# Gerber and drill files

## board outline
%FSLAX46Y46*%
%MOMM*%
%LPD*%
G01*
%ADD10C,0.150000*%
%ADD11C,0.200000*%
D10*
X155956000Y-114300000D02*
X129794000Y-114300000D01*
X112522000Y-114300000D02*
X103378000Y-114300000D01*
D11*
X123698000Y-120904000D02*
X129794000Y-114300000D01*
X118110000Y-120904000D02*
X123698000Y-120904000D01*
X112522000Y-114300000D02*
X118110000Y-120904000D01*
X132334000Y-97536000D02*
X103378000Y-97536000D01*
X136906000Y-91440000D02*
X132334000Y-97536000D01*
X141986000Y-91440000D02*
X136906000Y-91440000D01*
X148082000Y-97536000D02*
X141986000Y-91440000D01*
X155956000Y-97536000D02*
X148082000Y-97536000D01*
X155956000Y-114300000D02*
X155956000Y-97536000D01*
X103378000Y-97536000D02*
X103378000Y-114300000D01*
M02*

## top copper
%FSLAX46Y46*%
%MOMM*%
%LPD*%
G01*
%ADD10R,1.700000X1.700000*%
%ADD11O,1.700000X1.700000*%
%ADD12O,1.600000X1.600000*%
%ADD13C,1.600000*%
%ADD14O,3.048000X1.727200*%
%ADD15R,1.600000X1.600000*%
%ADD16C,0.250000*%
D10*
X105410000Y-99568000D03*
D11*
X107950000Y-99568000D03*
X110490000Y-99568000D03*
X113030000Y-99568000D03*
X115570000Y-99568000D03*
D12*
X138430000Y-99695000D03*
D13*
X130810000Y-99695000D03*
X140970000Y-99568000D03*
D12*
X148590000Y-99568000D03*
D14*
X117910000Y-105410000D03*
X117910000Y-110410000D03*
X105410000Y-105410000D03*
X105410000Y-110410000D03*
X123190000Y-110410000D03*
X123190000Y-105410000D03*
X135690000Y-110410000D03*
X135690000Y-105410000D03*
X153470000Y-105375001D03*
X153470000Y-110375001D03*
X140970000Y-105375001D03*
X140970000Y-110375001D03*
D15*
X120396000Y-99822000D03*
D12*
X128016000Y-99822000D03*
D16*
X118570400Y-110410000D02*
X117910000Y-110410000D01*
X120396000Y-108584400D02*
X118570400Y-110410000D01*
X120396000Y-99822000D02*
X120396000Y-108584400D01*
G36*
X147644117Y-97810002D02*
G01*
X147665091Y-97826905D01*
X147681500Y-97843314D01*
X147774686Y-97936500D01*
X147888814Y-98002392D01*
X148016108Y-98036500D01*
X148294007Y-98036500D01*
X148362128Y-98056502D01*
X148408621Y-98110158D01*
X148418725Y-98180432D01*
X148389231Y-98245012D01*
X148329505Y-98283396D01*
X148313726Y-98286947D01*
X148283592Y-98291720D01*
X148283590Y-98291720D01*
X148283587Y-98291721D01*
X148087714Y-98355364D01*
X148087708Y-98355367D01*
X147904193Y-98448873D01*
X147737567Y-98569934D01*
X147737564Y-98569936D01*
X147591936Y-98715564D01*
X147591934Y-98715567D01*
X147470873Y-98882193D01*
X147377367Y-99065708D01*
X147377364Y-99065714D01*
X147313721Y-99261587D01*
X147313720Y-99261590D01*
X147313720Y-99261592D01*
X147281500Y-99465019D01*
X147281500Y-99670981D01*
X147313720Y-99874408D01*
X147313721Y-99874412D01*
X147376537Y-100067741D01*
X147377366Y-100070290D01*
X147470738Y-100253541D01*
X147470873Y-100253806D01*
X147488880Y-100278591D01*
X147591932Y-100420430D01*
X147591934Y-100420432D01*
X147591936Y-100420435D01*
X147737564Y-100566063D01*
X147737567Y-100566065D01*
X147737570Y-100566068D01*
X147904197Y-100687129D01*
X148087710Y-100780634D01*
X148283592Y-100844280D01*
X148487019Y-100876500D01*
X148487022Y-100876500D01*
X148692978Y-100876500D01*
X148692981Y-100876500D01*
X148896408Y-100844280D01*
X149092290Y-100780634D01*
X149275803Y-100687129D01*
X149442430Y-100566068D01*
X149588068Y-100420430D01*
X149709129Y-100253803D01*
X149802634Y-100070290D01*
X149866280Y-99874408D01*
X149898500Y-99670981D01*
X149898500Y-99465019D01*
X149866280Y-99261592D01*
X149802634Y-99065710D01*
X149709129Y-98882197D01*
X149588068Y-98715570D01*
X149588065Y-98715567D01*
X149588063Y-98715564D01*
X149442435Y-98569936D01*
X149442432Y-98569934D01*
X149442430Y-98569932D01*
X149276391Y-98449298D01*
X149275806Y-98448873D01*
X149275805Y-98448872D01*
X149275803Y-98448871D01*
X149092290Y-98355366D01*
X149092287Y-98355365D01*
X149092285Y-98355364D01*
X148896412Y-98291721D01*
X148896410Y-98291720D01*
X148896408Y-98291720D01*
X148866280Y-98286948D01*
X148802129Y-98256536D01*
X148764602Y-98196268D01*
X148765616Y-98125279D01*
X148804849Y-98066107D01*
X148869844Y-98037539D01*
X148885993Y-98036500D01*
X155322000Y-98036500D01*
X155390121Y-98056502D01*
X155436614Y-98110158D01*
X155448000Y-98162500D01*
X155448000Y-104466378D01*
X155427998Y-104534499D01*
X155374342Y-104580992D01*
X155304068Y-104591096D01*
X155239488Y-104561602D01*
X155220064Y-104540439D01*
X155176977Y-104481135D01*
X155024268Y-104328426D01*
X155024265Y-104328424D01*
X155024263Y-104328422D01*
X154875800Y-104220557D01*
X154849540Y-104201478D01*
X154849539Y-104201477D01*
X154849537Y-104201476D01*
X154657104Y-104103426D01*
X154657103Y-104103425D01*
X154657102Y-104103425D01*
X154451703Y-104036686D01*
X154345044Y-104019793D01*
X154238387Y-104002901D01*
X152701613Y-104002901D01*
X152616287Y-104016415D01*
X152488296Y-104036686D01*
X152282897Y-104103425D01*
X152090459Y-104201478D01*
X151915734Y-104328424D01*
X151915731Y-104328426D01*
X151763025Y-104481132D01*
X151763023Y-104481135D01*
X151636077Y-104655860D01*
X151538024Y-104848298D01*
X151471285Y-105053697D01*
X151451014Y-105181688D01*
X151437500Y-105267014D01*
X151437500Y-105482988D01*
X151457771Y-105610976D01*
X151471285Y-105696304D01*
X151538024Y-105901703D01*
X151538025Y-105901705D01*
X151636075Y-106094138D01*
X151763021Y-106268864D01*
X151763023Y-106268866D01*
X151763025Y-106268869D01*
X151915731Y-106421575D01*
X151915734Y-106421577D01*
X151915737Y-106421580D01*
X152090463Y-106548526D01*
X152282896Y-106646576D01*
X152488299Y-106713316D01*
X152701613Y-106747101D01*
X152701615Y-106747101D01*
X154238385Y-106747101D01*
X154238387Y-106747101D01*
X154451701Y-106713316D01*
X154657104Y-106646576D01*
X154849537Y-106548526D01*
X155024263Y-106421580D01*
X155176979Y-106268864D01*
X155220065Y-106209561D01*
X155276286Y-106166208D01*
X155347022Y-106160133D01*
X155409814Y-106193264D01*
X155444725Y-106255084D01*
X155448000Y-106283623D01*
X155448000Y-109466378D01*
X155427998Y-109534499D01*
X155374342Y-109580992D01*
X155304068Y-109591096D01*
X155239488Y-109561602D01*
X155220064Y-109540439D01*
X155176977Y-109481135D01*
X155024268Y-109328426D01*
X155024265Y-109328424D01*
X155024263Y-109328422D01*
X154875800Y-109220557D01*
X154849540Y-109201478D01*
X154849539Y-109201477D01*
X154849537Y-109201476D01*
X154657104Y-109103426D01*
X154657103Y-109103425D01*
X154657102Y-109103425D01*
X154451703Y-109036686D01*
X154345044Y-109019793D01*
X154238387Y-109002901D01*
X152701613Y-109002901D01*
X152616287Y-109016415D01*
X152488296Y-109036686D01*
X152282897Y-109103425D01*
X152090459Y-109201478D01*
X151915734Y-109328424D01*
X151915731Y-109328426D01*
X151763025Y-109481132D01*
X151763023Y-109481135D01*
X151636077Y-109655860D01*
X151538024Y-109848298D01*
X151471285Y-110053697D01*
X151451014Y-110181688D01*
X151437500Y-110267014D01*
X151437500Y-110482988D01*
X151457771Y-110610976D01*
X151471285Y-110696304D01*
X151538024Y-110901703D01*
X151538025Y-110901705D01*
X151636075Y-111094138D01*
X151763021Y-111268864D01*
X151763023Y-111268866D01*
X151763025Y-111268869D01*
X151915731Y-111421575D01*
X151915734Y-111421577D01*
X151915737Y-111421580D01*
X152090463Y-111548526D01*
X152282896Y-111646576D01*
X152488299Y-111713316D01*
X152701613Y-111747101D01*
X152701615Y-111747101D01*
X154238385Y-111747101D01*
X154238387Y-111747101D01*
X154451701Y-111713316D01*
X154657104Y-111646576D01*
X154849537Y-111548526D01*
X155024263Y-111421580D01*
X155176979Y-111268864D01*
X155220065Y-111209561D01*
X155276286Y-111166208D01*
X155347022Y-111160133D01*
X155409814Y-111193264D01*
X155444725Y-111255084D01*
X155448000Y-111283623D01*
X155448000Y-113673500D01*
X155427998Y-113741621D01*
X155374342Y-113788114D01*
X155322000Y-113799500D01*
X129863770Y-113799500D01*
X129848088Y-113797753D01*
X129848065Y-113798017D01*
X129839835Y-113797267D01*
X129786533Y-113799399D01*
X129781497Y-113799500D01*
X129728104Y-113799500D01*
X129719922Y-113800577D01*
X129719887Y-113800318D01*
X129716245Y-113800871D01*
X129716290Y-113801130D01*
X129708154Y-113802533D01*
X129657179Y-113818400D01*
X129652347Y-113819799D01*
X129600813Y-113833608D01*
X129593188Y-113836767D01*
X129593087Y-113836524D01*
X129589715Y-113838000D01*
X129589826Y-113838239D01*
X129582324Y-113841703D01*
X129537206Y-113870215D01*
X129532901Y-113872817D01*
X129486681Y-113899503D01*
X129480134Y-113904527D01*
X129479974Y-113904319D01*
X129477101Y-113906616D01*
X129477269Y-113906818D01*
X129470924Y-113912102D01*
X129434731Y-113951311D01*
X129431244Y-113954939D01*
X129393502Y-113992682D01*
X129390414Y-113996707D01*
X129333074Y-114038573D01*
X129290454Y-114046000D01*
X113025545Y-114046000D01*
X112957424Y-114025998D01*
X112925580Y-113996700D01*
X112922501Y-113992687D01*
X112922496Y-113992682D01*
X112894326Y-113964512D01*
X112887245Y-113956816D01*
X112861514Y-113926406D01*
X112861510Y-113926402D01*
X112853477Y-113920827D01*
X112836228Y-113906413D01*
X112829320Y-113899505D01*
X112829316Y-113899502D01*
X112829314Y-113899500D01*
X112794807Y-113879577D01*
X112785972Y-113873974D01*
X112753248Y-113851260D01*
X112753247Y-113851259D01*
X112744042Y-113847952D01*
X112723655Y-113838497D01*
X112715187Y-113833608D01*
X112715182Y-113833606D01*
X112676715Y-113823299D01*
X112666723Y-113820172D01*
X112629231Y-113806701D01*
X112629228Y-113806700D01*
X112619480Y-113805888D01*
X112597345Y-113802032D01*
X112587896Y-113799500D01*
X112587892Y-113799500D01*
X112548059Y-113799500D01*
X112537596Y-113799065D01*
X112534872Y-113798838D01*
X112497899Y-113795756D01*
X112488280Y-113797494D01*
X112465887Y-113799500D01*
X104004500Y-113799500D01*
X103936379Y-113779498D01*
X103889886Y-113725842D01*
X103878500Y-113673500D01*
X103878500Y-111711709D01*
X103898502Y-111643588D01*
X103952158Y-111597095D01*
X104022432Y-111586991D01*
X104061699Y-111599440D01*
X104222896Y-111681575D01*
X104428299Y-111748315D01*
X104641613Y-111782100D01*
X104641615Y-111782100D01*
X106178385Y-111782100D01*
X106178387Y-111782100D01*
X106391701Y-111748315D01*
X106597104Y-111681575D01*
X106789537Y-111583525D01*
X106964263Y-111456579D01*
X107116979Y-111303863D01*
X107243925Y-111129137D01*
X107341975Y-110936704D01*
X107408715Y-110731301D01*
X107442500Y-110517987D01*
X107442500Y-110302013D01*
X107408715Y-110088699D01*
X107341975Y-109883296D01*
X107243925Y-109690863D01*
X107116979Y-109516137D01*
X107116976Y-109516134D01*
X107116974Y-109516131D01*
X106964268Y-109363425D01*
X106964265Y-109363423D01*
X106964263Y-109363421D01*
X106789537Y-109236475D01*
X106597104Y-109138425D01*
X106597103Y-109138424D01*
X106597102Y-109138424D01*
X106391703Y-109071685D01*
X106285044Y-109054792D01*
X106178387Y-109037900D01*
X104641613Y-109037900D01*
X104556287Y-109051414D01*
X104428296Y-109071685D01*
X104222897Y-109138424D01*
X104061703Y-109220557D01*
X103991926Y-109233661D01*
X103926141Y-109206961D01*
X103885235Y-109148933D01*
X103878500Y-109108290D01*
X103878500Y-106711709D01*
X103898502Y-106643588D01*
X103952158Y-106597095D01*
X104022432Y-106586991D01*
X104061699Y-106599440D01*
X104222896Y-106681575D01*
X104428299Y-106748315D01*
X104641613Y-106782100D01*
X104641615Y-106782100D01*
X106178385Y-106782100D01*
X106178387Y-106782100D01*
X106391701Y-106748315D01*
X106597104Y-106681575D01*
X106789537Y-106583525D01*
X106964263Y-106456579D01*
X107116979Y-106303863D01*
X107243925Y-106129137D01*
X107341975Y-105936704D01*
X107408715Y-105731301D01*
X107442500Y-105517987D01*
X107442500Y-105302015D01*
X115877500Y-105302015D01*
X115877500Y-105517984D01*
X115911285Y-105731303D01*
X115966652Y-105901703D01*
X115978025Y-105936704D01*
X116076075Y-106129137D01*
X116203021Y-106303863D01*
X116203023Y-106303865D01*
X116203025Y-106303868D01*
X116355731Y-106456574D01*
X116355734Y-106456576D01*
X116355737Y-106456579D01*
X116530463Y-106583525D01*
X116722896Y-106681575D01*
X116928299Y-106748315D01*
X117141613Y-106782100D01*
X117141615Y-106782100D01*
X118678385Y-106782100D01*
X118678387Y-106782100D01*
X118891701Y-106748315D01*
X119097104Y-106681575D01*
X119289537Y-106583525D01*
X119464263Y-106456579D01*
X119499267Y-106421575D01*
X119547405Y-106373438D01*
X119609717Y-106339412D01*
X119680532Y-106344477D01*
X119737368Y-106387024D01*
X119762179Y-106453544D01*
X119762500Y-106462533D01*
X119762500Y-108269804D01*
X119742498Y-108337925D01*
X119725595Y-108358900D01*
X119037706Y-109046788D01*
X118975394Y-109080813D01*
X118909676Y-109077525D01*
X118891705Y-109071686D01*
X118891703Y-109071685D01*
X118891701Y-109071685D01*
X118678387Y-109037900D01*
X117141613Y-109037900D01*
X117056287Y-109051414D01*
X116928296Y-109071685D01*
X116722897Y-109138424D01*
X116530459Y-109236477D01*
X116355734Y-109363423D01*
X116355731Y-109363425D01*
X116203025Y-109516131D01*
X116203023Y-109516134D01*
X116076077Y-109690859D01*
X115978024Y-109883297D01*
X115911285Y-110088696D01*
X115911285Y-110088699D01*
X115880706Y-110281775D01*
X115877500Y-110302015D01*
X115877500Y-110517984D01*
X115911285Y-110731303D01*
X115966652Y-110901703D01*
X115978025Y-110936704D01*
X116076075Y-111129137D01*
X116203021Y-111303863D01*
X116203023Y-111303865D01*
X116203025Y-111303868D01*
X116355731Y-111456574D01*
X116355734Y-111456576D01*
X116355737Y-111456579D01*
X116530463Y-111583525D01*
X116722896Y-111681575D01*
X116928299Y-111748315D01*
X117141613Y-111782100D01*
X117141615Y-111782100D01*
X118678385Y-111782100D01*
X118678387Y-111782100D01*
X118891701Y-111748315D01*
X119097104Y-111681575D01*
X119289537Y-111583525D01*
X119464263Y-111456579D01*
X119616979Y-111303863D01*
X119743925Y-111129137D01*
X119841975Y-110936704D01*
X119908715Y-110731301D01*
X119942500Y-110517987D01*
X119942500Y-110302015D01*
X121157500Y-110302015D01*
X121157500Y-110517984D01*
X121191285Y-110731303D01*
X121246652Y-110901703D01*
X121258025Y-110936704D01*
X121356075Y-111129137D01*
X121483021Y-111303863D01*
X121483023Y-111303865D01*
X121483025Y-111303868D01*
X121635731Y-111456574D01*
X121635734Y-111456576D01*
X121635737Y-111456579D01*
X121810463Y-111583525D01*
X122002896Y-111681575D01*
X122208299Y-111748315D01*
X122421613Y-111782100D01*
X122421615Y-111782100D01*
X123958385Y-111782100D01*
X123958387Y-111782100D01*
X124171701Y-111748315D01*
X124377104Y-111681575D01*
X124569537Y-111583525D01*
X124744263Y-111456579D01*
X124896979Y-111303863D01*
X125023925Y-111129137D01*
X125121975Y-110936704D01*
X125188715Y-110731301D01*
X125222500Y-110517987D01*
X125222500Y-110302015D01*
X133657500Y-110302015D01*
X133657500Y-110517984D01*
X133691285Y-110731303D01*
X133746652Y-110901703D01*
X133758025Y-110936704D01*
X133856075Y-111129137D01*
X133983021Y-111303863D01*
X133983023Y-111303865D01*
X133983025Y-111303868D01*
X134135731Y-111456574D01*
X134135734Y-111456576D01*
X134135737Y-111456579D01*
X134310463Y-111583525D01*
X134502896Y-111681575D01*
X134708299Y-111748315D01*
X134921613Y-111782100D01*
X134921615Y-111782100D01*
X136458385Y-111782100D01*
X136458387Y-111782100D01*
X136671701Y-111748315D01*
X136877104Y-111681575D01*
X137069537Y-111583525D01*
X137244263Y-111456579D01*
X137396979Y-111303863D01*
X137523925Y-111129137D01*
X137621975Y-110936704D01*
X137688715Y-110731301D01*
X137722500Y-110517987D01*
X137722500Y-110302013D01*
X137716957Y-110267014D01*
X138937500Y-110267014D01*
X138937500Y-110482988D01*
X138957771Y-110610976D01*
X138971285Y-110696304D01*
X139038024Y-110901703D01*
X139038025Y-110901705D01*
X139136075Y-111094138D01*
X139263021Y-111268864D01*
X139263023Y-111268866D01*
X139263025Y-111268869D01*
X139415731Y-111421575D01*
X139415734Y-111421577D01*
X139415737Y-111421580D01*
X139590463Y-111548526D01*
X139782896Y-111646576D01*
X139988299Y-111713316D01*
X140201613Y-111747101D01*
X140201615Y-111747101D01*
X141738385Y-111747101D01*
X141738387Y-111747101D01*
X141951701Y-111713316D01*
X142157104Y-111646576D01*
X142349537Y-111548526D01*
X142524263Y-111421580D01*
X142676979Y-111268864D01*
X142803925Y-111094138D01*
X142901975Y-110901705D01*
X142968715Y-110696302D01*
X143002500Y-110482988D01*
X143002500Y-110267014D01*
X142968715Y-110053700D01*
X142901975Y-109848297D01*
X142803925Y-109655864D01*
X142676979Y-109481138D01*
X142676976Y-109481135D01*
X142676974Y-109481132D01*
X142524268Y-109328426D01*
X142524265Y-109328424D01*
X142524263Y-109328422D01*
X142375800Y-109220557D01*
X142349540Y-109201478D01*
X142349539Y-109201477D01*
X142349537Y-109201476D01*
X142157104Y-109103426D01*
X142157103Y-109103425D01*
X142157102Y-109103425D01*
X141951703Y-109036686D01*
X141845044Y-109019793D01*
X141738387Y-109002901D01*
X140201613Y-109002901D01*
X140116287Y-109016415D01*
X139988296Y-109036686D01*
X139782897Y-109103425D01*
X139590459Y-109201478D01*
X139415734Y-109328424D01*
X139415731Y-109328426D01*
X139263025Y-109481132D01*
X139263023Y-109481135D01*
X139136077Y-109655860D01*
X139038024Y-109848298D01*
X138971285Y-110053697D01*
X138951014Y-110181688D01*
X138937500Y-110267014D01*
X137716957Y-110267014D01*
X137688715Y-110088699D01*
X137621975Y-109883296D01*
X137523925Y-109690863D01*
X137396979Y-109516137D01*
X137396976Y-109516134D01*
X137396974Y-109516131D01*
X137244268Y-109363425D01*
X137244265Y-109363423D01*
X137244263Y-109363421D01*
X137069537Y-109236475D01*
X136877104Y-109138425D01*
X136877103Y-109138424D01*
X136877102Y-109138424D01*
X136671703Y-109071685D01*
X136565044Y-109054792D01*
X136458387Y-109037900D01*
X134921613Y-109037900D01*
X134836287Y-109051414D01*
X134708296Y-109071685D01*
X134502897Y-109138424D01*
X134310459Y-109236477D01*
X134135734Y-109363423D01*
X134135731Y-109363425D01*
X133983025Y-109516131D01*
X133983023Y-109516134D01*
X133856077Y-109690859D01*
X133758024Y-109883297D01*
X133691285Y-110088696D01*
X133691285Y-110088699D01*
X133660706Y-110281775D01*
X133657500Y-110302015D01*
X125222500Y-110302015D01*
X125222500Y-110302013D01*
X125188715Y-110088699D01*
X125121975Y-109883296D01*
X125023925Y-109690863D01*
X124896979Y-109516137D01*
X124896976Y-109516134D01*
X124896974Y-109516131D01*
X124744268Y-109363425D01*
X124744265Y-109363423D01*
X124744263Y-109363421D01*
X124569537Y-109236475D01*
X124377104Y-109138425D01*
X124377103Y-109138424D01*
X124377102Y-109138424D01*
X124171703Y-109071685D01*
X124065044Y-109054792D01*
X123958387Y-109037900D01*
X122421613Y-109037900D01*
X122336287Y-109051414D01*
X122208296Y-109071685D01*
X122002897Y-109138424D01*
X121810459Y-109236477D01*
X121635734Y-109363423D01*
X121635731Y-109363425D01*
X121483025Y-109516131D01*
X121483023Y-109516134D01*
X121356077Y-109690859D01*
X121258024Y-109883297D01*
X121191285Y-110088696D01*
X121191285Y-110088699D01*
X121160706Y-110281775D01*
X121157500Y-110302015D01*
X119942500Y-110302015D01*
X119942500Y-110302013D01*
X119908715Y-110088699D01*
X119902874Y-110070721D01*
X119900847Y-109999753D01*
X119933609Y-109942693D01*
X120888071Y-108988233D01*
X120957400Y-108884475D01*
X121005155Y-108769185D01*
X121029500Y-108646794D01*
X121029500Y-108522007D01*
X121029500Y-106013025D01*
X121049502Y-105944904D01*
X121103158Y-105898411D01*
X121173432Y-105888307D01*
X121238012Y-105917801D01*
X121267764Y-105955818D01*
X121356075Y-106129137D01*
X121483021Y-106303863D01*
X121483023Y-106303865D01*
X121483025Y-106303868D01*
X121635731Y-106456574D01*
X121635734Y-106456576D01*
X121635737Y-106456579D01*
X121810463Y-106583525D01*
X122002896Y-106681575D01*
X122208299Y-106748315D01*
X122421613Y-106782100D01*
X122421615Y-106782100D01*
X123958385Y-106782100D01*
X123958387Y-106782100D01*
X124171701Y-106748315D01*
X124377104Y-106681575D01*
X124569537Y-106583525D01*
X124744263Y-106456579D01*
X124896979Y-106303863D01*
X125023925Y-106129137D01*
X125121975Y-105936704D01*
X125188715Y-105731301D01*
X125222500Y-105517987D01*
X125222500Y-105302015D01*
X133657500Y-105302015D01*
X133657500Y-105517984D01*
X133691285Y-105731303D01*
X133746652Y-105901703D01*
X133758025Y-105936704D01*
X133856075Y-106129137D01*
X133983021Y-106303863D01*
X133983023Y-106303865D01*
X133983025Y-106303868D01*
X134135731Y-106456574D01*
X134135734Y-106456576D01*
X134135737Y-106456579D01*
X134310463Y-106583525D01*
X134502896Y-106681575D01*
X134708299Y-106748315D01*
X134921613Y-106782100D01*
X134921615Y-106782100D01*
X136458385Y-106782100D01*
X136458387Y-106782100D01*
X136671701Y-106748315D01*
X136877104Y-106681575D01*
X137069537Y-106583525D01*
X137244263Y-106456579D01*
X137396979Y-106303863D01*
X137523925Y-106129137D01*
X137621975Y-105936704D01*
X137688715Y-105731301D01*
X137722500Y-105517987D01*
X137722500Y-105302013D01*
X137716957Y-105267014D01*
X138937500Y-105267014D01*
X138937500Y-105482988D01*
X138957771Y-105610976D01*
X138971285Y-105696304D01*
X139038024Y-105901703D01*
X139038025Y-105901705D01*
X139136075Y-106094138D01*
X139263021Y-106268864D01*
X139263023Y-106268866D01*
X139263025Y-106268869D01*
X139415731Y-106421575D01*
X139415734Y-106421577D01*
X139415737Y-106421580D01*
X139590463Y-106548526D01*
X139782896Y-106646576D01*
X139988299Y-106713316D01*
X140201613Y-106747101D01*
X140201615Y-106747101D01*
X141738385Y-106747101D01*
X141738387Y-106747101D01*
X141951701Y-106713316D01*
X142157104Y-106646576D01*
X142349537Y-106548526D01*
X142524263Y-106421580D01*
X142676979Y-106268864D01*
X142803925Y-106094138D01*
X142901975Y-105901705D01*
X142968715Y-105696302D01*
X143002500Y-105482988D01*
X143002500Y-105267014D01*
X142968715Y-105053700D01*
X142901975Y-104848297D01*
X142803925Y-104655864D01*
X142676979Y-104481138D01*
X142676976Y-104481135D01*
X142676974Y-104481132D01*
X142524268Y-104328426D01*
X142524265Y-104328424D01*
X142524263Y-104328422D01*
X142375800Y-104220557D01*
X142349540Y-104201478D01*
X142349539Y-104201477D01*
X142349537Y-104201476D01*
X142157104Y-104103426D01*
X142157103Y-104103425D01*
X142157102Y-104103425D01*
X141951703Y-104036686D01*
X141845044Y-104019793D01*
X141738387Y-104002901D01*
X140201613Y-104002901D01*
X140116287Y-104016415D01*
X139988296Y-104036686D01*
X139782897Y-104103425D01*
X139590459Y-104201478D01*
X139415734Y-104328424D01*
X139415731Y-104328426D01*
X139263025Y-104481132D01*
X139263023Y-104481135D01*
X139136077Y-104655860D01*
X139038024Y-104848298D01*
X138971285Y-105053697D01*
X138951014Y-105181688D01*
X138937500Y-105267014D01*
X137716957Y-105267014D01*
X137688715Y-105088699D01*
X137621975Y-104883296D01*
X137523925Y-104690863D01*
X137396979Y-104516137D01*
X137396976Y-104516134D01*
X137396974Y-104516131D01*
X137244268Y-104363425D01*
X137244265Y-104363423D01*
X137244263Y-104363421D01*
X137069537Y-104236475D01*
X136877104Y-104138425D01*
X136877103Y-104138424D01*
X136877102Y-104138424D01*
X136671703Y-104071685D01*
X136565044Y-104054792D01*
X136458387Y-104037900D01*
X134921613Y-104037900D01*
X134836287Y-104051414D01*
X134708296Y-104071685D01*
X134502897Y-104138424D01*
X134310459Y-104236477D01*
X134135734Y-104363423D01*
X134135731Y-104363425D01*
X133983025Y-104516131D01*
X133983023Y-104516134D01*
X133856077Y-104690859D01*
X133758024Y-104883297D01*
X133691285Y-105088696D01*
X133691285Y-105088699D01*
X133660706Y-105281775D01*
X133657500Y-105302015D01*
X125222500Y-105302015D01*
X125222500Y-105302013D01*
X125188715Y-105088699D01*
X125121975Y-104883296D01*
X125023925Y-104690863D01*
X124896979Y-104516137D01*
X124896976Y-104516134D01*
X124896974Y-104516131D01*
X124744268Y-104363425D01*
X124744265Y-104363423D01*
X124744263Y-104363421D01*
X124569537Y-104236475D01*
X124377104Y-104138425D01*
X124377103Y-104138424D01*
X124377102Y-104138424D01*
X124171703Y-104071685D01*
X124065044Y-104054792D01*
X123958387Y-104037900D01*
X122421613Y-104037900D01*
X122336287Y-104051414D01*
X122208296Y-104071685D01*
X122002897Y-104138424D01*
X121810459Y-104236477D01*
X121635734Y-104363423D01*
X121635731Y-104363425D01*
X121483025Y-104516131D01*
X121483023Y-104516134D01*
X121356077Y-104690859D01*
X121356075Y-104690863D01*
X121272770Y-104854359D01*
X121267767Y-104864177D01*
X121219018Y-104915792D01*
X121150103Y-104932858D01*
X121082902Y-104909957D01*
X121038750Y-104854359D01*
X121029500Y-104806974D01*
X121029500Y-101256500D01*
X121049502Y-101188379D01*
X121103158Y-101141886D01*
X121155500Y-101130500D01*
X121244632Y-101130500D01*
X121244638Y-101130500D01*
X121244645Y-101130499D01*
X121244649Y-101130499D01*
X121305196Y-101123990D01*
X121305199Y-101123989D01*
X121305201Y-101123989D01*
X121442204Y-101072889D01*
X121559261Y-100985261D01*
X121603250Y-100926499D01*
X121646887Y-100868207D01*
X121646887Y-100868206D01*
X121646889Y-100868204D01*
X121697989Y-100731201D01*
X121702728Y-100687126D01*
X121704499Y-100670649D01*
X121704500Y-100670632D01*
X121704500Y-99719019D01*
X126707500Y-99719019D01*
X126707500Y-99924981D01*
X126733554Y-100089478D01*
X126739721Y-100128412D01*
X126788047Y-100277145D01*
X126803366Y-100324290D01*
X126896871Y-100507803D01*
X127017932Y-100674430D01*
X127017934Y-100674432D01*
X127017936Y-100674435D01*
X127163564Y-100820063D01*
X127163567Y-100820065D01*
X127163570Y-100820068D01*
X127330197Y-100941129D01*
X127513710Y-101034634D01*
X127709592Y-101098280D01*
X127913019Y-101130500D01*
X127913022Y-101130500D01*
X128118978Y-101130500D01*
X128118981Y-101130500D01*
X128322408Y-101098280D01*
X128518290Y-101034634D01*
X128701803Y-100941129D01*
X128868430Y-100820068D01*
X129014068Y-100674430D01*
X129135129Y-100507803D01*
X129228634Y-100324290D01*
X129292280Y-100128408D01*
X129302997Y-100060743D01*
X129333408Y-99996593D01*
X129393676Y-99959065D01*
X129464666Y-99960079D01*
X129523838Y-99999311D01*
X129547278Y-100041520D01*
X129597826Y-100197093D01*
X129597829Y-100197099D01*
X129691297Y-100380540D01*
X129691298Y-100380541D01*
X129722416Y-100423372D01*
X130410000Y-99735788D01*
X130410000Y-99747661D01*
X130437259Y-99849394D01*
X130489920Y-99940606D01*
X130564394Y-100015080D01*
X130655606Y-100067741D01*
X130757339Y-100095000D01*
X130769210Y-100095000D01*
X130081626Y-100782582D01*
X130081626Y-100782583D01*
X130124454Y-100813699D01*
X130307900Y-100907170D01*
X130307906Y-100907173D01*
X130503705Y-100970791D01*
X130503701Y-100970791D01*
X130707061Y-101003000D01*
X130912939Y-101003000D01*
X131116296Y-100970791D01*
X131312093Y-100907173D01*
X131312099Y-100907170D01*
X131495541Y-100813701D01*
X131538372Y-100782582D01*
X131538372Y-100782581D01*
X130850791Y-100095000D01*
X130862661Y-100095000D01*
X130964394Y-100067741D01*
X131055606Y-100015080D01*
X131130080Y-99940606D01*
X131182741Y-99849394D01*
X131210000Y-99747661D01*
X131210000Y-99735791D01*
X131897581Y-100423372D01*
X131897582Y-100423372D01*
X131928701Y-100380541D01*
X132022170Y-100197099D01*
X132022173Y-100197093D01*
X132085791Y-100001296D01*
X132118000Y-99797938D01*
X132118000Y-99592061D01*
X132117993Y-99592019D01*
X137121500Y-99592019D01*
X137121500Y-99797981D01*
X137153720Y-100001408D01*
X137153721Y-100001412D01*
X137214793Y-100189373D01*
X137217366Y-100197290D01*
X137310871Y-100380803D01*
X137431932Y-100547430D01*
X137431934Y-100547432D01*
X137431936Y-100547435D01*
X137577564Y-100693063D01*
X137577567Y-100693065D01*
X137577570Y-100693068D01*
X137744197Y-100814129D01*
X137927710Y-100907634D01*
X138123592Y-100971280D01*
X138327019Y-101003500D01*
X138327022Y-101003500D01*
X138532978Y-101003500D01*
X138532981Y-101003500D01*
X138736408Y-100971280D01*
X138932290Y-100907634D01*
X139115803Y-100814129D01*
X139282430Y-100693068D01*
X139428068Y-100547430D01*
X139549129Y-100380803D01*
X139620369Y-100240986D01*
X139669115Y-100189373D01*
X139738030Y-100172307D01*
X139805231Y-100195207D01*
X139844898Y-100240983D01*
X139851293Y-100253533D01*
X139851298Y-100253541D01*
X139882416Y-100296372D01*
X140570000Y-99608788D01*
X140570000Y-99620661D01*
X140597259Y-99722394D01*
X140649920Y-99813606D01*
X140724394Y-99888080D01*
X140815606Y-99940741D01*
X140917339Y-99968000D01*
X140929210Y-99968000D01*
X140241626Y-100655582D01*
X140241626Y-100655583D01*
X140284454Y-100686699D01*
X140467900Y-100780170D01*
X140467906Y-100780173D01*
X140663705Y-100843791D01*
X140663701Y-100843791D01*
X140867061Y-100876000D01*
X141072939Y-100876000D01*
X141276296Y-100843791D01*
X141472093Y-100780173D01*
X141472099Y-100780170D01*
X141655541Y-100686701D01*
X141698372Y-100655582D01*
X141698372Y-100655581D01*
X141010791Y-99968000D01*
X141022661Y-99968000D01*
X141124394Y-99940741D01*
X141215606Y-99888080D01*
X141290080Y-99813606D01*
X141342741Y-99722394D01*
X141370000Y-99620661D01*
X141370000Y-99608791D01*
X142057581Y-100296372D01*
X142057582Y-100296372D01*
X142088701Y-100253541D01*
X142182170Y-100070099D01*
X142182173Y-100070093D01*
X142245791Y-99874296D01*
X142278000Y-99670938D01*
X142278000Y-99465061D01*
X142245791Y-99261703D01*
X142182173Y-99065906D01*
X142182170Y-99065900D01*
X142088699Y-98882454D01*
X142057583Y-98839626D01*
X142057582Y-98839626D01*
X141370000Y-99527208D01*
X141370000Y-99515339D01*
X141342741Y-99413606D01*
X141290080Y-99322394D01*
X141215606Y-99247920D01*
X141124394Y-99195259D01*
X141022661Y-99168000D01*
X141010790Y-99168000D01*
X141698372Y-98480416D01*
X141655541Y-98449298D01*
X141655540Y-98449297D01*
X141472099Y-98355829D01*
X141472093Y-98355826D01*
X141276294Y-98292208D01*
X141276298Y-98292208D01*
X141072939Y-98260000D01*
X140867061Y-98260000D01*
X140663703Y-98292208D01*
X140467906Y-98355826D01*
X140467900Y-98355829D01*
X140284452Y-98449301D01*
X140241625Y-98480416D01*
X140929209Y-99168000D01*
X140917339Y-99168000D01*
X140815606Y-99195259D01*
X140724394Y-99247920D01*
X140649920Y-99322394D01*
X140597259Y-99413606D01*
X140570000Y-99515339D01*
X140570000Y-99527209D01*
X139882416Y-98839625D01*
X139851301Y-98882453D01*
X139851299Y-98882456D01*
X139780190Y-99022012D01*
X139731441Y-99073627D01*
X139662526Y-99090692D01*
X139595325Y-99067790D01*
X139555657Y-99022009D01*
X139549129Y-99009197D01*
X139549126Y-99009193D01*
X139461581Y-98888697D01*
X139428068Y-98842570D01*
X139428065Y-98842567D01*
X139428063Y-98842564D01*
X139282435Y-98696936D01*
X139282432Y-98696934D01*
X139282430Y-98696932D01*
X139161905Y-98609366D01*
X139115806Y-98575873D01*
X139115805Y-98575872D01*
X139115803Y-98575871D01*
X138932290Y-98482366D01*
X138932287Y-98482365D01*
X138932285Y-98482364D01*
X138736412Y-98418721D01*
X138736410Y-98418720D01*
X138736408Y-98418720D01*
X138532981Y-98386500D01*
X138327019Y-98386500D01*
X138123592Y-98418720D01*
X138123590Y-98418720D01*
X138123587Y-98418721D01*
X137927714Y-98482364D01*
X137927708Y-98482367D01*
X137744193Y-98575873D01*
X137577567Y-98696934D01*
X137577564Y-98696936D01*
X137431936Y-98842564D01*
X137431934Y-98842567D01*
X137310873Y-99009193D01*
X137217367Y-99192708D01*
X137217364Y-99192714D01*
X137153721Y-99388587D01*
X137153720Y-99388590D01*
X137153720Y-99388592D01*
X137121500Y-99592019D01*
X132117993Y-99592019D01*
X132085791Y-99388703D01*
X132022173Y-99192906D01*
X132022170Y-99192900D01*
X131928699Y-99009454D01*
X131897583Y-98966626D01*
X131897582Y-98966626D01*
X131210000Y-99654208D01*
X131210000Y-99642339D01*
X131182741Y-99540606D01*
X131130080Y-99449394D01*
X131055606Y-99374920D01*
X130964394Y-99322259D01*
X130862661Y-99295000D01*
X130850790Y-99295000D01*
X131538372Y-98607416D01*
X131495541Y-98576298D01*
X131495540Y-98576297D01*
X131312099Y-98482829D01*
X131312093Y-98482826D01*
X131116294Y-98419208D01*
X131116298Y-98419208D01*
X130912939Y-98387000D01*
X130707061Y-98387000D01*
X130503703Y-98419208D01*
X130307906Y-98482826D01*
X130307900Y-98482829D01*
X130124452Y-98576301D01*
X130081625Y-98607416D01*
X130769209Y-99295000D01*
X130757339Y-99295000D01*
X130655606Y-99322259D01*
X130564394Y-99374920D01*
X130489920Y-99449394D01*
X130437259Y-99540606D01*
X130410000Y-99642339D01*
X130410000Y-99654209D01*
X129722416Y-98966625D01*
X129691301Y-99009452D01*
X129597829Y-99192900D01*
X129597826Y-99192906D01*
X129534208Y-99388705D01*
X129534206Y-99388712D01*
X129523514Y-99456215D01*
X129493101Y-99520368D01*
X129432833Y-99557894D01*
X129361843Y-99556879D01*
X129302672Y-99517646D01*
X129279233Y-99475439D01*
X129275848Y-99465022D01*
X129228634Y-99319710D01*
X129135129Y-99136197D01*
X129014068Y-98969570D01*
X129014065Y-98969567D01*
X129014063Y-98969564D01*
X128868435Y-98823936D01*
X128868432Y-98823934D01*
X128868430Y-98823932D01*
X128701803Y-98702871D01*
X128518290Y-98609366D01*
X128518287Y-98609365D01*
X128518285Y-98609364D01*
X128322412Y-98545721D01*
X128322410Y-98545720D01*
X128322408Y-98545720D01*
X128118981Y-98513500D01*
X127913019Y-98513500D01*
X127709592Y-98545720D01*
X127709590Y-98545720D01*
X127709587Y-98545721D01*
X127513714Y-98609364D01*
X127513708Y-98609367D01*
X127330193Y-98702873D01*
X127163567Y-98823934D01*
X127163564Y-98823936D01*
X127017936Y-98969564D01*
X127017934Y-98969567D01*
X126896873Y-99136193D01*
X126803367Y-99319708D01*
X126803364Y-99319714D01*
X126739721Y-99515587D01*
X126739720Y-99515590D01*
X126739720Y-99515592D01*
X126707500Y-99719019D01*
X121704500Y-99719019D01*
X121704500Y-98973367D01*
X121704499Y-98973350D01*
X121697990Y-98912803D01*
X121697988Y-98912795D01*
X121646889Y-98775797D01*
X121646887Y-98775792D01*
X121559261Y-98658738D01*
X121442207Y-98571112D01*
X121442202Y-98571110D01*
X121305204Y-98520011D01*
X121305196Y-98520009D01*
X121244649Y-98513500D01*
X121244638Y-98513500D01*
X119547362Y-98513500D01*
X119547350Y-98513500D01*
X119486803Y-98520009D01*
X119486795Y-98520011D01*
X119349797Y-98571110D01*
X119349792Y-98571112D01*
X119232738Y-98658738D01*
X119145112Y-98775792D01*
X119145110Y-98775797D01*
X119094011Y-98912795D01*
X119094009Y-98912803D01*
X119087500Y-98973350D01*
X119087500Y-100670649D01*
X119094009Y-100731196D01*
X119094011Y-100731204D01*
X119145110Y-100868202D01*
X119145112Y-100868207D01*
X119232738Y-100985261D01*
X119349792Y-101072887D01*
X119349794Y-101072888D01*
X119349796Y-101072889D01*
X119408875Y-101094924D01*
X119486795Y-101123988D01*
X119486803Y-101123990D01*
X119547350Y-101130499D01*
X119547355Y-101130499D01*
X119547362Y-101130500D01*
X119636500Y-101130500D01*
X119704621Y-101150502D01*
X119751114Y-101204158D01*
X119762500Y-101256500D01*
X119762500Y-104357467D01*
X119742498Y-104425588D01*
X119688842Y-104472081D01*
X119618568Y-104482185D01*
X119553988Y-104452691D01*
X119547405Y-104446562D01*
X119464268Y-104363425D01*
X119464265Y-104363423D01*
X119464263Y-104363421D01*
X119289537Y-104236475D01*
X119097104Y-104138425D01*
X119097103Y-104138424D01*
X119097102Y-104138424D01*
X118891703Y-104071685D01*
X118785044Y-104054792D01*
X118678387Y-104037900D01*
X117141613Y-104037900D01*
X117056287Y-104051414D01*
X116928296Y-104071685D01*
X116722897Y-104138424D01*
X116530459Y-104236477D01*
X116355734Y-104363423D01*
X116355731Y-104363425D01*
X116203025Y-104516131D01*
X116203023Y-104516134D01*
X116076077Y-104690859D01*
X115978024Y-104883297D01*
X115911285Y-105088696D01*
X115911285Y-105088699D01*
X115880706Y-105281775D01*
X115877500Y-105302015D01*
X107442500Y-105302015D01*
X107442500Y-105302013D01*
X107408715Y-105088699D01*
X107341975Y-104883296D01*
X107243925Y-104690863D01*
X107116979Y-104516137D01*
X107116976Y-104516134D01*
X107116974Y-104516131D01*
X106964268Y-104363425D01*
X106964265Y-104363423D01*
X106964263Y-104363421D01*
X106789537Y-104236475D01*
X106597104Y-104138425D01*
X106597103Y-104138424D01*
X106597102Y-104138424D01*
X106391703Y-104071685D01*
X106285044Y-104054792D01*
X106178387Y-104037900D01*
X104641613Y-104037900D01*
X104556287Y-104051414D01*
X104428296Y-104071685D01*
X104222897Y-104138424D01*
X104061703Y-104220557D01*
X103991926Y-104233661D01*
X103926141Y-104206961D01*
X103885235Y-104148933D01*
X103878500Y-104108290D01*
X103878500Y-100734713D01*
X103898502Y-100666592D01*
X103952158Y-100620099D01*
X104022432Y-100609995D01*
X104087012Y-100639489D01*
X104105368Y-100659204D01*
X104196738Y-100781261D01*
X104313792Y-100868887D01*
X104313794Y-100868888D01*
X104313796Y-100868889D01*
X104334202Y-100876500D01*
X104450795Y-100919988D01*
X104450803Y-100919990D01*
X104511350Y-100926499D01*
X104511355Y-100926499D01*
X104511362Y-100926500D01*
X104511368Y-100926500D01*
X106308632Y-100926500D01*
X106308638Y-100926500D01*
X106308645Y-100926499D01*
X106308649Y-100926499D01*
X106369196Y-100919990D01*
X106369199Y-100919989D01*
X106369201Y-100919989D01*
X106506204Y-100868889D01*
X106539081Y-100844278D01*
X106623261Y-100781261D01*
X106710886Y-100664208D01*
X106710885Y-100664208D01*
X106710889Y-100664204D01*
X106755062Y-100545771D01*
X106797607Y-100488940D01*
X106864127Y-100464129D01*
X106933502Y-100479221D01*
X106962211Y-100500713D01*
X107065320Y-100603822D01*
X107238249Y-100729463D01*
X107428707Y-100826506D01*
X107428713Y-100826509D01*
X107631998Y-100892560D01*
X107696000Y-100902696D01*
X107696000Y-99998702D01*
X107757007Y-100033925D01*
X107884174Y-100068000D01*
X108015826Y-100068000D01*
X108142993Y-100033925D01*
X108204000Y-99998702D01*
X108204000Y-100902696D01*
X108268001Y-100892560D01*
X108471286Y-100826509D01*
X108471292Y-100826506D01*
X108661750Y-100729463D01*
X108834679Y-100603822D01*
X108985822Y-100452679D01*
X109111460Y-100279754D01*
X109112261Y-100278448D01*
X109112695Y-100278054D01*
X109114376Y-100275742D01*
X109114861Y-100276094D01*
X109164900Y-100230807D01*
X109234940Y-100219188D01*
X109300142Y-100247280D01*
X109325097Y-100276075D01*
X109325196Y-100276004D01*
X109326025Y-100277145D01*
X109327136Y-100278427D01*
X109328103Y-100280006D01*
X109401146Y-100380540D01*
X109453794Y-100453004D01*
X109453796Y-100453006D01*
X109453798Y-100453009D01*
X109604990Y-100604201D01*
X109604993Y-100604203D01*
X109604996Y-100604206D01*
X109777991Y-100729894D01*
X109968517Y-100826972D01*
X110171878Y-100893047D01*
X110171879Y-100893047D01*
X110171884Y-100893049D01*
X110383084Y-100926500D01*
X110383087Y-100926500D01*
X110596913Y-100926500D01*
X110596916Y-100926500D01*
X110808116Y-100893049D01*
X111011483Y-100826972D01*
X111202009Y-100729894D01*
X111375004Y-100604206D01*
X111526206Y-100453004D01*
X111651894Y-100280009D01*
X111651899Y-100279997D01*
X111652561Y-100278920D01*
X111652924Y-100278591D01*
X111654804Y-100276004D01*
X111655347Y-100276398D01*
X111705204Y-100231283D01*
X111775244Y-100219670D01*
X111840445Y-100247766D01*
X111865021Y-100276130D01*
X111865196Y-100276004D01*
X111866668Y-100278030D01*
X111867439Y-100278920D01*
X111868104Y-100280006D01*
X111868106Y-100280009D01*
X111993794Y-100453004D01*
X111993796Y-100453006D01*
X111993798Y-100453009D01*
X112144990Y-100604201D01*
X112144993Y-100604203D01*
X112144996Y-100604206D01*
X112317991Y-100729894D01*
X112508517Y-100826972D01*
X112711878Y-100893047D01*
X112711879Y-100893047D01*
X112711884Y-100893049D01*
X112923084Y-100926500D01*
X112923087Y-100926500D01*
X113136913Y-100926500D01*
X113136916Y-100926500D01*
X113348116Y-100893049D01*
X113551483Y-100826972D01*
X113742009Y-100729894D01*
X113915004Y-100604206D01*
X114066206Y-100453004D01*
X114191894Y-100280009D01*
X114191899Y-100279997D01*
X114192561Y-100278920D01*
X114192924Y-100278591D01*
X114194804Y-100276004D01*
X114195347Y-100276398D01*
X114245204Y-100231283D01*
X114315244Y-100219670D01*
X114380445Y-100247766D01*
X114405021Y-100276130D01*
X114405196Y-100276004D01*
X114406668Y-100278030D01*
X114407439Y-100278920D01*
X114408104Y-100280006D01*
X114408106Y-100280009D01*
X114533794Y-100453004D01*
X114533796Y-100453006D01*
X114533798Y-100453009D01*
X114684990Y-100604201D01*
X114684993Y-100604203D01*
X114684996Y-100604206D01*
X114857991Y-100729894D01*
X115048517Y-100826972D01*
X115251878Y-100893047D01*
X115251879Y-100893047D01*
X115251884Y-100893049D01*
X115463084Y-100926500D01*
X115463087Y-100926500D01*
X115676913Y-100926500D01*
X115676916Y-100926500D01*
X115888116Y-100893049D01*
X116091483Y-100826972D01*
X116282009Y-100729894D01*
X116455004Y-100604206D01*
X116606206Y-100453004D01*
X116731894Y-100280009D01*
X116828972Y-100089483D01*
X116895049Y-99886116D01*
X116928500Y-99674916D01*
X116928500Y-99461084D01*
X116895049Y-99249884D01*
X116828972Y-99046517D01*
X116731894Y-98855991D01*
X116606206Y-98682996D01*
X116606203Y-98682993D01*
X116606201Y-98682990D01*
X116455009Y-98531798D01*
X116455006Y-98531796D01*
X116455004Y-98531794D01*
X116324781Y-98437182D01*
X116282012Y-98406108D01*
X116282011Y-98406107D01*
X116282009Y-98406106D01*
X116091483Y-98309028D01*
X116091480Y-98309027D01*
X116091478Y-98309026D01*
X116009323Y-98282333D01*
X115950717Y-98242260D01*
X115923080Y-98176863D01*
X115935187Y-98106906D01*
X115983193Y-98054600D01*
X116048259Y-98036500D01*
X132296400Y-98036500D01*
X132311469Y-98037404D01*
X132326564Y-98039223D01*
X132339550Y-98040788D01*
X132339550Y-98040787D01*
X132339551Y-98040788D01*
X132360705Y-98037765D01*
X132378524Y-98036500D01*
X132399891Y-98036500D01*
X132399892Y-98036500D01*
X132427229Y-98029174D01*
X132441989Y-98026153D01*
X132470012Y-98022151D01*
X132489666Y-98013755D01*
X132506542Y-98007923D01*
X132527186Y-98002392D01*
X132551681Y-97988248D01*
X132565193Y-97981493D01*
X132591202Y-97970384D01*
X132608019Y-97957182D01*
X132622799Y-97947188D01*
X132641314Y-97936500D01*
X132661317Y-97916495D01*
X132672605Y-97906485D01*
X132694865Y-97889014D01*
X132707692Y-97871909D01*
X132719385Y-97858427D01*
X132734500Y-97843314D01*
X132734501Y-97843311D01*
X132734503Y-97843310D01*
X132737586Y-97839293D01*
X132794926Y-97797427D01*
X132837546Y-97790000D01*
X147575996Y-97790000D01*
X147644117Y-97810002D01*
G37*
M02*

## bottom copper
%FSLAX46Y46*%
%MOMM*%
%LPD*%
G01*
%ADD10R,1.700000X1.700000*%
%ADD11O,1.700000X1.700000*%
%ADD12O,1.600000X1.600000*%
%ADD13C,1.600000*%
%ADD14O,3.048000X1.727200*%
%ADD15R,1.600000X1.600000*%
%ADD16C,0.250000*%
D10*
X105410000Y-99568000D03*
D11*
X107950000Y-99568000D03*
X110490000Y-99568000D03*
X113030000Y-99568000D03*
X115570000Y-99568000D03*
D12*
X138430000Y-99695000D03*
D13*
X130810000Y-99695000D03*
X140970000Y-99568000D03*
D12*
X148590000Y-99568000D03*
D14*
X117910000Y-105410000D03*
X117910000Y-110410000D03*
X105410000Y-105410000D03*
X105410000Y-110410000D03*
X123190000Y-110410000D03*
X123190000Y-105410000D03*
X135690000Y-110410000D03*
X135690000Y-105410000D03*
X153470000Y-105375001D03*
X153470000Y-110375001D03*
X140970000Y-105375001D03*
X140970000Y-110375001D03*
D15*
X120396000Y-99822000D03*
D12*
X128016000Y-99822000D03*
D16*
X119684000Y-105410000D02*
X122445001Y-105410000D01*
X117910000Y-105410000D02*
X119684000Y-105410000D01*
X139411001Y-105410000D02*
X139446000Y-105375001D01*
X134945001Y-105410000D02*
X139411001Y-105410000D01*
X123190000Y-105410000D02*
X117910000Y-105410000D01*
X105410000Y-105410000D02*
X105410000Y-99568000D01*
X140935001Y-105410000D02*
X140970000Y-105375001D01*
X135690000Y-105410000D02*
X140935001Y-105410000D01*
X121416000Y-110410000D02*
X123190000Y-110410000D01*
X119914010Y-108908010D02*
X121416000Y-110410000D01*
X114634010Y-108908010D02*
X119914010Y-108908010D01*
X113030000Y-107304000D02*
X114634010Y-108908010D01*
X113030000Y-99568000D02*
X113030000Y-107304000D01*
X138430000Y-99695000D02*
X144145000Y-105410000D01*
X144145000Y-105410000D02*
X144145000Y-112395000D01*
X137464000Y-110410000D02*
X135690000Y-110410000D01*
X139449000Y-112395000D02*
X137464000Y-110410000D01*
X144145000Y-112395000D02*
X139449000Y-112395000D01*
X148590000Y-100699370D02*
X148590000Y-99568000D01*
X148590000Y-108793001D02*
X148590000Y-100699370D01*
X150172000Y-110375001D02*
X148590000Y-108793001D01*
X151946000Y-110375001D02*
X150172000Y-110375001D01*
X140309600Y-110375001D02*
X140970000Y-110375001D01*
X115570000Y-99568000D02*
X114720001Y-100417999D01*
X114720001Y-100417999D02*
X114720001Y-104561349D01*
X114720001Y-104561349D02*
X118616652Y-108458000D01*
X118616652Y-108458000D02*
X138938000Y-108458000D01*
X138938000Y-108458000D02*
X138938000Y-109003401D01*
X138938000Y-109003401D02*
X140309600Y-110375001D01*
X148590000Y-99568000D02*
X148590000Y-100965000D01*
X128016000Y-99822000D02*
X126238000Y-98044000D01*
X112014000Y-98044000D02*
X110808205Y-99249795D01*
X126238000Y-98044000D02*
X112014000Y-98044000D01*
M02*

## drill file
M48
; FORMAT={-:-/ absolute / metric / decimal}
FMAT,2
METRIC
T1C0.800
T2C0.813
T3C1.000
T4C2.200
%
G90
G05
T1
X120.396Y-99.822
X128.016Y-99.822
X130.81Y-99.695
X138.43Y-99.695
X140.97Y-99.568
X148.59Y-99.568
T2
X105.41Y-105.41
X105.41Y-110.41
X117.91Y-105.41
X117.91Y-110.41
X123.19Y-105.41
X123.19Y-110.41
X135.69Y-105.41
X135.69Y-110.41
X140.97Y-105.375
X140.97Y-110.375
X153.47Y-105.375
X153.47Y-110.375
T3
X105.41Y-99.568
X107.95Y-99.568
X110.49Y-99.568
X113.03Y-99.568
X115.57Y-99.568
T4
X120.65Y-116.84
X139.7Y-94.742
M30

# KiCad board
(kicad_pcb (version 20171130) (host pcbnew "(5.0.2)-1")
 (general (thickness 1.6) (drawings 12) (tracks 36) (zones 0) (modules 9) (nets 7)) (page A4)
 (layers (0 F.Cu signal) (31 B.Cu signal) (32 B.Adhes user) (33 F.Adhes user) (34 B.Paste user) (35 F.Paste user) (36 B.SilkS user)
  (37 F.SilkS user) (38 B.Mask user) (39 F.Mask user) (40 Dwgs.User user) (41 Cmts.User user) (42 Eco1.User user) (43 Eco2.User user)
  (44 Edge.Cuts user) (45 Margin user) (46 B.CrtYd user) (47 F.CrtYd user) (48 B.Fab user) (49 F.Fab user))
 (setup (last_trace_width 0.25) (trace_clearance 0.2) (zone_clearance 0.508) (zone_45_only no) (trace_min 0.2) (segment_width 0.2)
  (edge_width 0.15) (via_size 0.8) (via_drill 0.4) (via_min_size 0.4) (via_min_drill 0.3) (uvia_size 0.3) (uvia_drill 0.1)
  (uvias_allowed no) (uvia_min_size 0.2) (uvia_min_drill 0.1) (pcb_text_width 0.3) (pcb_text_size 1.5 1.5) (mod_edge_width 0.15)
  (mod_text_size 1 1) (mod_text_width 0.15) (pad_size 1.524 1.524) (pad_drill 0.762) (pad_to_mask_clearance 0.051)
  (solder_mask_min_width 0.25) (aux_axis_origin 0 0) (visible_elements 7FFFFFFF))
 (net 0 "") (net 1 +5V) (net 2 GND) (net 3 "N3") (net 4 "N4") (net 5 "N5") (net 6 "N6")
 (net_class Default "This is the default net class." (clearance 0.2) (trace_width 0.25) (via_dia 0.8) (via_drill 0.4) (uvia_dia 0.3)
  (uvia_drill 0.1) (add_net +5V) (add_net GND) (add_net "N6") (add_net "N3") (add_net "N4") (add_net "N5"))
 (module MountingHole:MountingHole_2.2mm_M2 (layer F.Cu) (at 139.7 94.742)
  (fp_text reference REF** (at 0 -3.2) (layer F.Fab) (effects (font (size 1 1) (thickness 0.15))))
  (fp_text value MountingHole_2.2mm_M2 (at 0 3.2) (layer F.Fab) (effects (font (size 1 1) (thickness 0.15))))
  (pad 1 np_thru_hole circle (at 0 0) (size 2.2 2.2) (drill 2.2) (layers *.Cu *.Mask)))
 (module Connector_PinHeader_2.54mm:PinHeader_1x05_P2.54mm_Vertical (layer F.Cu) (at 105.41 99.568 90)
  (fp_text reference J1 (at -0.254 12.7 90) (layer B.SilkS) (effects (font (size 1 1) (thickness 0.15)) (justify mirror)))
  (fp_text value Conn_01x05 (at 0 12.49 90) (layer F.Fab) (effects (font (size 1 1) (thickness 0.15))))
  (pad 1 thru_hole rect (at 0 0 90) (size 1.7 1.7) (drill 1) (layers *.Cu *.Mask) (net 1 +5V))
  (pad 2 thru_hole oval (at 0 2.54 90) (size 1.7 1.7) (drill 1) (layers *.Cu *.Mask) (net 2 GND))
  (pad 3 thru_hole oval (at 0 5.08 90) (size 1.7 1.7) (drill 1) (layers *.Cu *.Mask) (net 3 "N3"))
  (pad 4 thru_hole oval (at 0 7.62 90) (size 1.7 1.7) (drill 1) (layers *.Cu *.Mask) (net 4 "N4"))
  (pad 5 thru_hole oval (at 0 10.16 90) (size 1.7 1.7) (drill 1) (layers *.Cu *.Mask) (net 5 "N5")))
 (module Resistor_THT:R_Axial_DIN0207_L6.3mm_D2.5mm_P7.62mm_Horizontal (layer F.Cu) (at 130.81 99.695)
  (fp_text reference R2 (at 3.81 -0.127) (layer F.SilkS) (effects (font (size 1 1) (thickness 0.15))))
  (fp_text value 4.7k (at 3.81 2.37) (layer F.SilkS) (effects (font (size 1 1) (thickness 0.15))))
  (pad 2 thru_hole oval (at 7.62 0) (size 1.6 1.6) (drill 0.8) (layers *.Cu *.Mask) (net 4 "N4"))
  (pad 1 thru_hole circle (at 0 0) (size 1.6 1.6) (drill 0.8) (layers *.Cu *.Mask) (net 2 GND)))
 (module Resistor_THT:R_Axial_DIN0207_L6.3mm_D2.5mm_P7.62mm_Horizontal (layer F.Cu) (at 140.97 99.568)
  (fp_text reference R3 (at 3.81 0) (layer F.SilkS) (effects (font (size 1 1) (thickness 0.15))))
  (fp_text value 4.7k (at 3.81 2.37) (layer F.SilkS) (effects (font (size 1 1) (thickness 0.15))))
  (pad 1 thru_hole circle (at 0 0) (size 1.6 1.6) (drill 0.8) (layers *.Cu *.Mask) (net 2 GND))
  (pad 2 thru_hole oval (at 7.62 0) (size 1.6 1.6) (drill 0.8) (layers *.Cu *.Mask) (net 5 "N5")))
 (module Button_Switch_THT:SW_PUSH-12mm (layer F.Cu) (at 105.41 105.41)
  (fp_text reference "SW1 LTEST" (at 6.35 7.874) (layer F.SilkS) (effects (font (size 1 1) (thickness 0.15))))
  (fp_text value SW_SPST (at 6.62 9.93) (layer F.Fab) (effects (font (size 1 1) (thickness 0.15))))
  (pad 1 thru_hole oval (at 12.5 0) (size 3.048 1.7272) (drill 0.8128) (layers *.Cu *.Mask) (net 1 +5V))
  (pad 2 thru_hole oval (at 12.5 5) (size 3.048 1.7272) (drill 0.8128) (layers *.Cu *.Mask) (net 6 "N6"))
  (pad 1 thru_hole oval (at 0 0) (size 3.048 1.7272) (drill 0.8128) (layers *.Cu *.Mask) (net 1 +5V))
  (pad 2 thru_hole oval (at 0 5) (size 3.048 1.7272) (drill 0.8128) (layers *.Cu *.Mask) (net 6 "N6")))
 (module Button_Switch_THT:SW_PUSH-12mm (layer F.Cu) (at 123.19 105.41)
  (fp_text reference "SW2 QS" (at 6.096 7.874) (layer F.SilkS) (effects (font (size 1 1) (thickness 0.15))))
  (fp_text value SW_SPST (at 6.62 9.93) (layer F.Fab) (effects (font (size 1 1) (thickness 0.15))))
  (pad 2 thru_hole oval (at 0 5) (size 3.048 1.7272) (drill 0.8128) (layers *.Cu *.Mask) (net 4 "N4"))
  (pad 1 thru_hole oval (at 0 0) (size 3.048 1.7272) (drill 0.8128) (layers *.Cu *.Mask) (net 1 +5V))
  (pad 2 thru_hole oval (at 12.5 5) (size 3.048 1.7272) (drill 0.8128) (layers *.Cu *.Mask) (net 4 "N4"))
  (pad 1 thru_hole oval (at 12.5 0) (size 3.048 1.7272) (drill 0.8128) (layers *.Cu *.Mask) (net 1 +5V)))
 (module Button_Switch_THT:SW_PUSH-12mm (layer F.Cu) (at 140.97 105.375001)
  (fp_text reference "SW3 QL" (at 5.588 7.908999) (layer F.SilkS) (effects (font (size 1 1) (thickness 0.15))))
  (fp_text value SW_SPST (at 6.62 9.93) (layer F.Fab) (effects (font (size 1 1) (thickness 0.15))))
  (pad 1 thru_hole oval (at 12.5 0) (size 3.048 1.7272) (drill 0.8128) (layers *.Cu *.Mask) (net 1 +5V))
  (pad 2 thru_hole oval (at 12.5 5) (size 3.048 1.7272) (drill 0.8128) (layers *.Cu *.Mask) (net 5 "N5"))
  (pad 1 thru_hole oval (at 0 0) (size 3.048 1.7272) (drill 0.8128) (layers *.Cu *.Mask) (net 1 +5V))
  (pad 2 thru_hole oval (at 0 5) (size 3.048 1.7272) (drill 0.8128) (layers *.Cu *.Mask) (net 5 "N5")))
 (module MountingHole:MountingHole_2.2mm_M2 (layer F.Cu) (at 120.65 116.84)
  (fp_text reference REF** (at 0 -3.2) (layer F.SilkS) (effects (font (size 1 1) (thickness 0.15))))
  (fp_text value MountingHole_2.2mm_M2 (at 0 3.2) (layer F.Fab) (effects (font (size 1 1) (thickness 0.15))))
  (pad 1 np_thru_hole circle (at 0 0) (size 2.2 2.2) (drill 2.2) (layers *.Cu *.Mask)))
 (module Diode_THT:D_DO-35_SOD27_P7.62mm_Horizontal (layer F.Cu) (at 120.396 99.822)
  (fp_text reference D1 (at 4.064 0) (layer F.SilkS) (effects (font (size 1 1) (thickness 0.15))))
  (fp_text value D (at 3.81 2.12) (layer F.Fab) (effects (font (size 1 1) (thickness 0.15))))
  (pad 1 thru_hole rect (at 0 0) (size 1.6 1.6) (drill 0.8) (layers *.Cu *.Mask) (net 6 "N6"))
  (pad 2 thru_hole oval (at 7.62 0) (size 1.6 1.6) (drill 0.8) (layers *.Cu *.Mask) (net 3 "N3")))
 (gr_line (start 155.956 114.3) (end 129.794 114.3) (layer Edge.Cuts) (width 0.15))
 (gr_line (start 112.522 114.3) (end 103.378 114.3) (layer Edge.Cuts) (width 0.15))
 (gr_line (start 123.698 120.904) (end 129.794 114.3) (layer Edge.Cuts) (width 0.2))
 (gr_line (start 118.11 120.904) (end 123.698 120.904) (layer Edge.Cuts) (width 0.2))
 (gr_line (start 112.522 114.3) (end 118.11 120.904) (layer Edge.Cuts) (width 0.2))
 (gr_line (start 132.334 97.536) (end 103.378 97.536) (layer Edge.Cuts) (width 0.2))
 (gr_line (start 136.906 91.44) (end 132.334 97.536) (layer Edge.Cuts) (width 0.2))
 (gr_line (start 141.986 91.44) (end 136.906 91.44) (layer Edge.Cuts) (width 0.2))
 (gr_line (start 148.082 97.536) (end 141.986 91.44) (layer Edge.Cuts) (width 0.2))
 (gr_line (start 155.956 97.536) (end 148.082 97.536) (layer Edge.Cuts) (width 0.2))
 (gr_line (start 155.956 114.3) (end 155.956 97.536) (layer Edge.Cuts) (width 0.2))
 (gr_line (start 103.378 97.536) (end 103.378 114.3) (layer Edge.Cuts) (width 0.2))
 (segment (start 119.684 105.41) (end 122.445001 105.41) (width 0.25) (layer B.Cu) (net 1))
 (segment (start 117.91 105.41) (end 119.684 105.41) (width 0.25) (layer B.Cu) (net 1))
 (segment (start 139.411001 105.41) (end 139.446 105.375001) (width 0.25) (layer B.Cu) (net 1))
 (segment (start 134.945001 105.41) (end 139.411001 105.41) (width 0.25) (layer B.Cu) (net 1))
 (segment (start 123.19 105.41) (end 117.91 105.41) (width 0.25) (layer B.Cu) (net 1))
 (segment (start 105.41 105.41) (end 105.41 99.568) (width 0.25) (layer B.Cu) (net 1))
 (segment (start 140.935001 105.41) (end 140.97 105.375001) (width 0.25) (layer B.Cu) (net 1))
 (segment (start 135.69 105.41) (end 140.935001 105.41) (width 0.25) (layer B.Cu) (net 1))
 (segment (start 121.416 110.41) (end 123.19 110.41) (width 0.25) (layer B.Cu) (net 4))
 (segment (start 119.91401 108.90801) (end 121.416 110.41) (width 0.25) (layer B.Cu) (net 4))
 (segment (start 114.63401 108.90801) (end 119.91401 108.90801) (width 0.25) (layer B.Cu) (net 4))
 (segment (start 113.03 107.304) (end 114.63401 108.90801) (width 0.25) (layer B.Cu) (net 4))
 (segment (start 113.03 99.568) (end 113.03 107.304) (width 0.25) (layer B.Cu) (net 4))
 (segment (start 138.43 99.695) (end 144.145 105.41) (width 0.25) (layer B.Cu) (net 4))
 (segment (start 144.145 105.41) (end 144.145 112.395) (width 0.25) (layer B.Cu) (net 4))
 (segment (start 137.464 110.41) (end 135.69 110.41) (width 0.25) (layer B.Cu) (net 4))
 (segment (start 139.449 112.395) (end 137.464 110.41) (width 0.25) (layer B.Cu) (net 4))
 (segment (start 144.145 112.395) (end 139.449 112.395) (width 0.25) (layer B.Cu) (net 4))
 (segment (start 148.59 100.69937) (end 148.59 99.568) (width 0.25) (layer B.Cu) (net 5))
 (segment (start 148.59 108.793001) (end 148.59 100.69937) (width 0.25) (layer B.Cu) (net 5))
 (segment (start 150.172 110.375001) (end 148.59 108.793001) (width 0.25) (layer B.Cu) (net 5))
 (segment (start 151.946 110.375001) (end 150.172 110.375001) (width 0.25) (layer B.Cu) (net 5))
 (segment (start 140.3096 110.375001) (end 140.97 110.375001) (width 0.25) (layer B.Cu) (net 5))
 (segment (start 115.57 99.568) (end 114.720001 100.417999) (width 0.25) (layer B.Cu) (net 5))
 (segment (start 114.720001 100.417999) (end 114.720001 104.561349) (width 0.25) (layer B.Cu) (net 5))
 (segment (start 114.720001 104.561349) (end 118.616652 108.458) (width 0.25) (layer B.Cu) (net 5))
 (segment (start 118.616652 108.458) (end 138.938 108.458) (width 0.25) (layer B.Cu) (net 5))
 (segment (start 138.938 108.458) (end 138.938 109.003401) (width 0.25) (layer B.Cu) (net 5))
 (segment (start 138.938 109.003401) (end 140.3096 110.375001) (width 0.25) (layer B.Cu) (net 5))
 (segment (start 148.59 99.568) (end 148.59 100.965) (width 0.25) (layer B.Cu) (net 5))
 (segment (start 118.5704 110.41) (end 117.91 110.41) (width 0.25) (layer F.Cu) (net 6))
 (segment (start 120.396 108.5844) (end 118.5704 110.41) (width 0.25) (layer F.Cu) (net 6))
 (segment (start 120.396 99.822) (end 120.396 108.5844) (width 0.25) (layer F.Cu) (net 6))
 (segment (start 128.016 99.822) (end 126.238 98.044) (width 0.25) (layer B.Cu) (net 3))
 (segment (start 112.014 98.044) (end 110.808205 99.249795) (width 0.25) (layer B.Cu) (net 3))
 (segment (start 126.238 98.044) (end 112.014 98.044) (width 0.25) (layer B.Cu) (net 3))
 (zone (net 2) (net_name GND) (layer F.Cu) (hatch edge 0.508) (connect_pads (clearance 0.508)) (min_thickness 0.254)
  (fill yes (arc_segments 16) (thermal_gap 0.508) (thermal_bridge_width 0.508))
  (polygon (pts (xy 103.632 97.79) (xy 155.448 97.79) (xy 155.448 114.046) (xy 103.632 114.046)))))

